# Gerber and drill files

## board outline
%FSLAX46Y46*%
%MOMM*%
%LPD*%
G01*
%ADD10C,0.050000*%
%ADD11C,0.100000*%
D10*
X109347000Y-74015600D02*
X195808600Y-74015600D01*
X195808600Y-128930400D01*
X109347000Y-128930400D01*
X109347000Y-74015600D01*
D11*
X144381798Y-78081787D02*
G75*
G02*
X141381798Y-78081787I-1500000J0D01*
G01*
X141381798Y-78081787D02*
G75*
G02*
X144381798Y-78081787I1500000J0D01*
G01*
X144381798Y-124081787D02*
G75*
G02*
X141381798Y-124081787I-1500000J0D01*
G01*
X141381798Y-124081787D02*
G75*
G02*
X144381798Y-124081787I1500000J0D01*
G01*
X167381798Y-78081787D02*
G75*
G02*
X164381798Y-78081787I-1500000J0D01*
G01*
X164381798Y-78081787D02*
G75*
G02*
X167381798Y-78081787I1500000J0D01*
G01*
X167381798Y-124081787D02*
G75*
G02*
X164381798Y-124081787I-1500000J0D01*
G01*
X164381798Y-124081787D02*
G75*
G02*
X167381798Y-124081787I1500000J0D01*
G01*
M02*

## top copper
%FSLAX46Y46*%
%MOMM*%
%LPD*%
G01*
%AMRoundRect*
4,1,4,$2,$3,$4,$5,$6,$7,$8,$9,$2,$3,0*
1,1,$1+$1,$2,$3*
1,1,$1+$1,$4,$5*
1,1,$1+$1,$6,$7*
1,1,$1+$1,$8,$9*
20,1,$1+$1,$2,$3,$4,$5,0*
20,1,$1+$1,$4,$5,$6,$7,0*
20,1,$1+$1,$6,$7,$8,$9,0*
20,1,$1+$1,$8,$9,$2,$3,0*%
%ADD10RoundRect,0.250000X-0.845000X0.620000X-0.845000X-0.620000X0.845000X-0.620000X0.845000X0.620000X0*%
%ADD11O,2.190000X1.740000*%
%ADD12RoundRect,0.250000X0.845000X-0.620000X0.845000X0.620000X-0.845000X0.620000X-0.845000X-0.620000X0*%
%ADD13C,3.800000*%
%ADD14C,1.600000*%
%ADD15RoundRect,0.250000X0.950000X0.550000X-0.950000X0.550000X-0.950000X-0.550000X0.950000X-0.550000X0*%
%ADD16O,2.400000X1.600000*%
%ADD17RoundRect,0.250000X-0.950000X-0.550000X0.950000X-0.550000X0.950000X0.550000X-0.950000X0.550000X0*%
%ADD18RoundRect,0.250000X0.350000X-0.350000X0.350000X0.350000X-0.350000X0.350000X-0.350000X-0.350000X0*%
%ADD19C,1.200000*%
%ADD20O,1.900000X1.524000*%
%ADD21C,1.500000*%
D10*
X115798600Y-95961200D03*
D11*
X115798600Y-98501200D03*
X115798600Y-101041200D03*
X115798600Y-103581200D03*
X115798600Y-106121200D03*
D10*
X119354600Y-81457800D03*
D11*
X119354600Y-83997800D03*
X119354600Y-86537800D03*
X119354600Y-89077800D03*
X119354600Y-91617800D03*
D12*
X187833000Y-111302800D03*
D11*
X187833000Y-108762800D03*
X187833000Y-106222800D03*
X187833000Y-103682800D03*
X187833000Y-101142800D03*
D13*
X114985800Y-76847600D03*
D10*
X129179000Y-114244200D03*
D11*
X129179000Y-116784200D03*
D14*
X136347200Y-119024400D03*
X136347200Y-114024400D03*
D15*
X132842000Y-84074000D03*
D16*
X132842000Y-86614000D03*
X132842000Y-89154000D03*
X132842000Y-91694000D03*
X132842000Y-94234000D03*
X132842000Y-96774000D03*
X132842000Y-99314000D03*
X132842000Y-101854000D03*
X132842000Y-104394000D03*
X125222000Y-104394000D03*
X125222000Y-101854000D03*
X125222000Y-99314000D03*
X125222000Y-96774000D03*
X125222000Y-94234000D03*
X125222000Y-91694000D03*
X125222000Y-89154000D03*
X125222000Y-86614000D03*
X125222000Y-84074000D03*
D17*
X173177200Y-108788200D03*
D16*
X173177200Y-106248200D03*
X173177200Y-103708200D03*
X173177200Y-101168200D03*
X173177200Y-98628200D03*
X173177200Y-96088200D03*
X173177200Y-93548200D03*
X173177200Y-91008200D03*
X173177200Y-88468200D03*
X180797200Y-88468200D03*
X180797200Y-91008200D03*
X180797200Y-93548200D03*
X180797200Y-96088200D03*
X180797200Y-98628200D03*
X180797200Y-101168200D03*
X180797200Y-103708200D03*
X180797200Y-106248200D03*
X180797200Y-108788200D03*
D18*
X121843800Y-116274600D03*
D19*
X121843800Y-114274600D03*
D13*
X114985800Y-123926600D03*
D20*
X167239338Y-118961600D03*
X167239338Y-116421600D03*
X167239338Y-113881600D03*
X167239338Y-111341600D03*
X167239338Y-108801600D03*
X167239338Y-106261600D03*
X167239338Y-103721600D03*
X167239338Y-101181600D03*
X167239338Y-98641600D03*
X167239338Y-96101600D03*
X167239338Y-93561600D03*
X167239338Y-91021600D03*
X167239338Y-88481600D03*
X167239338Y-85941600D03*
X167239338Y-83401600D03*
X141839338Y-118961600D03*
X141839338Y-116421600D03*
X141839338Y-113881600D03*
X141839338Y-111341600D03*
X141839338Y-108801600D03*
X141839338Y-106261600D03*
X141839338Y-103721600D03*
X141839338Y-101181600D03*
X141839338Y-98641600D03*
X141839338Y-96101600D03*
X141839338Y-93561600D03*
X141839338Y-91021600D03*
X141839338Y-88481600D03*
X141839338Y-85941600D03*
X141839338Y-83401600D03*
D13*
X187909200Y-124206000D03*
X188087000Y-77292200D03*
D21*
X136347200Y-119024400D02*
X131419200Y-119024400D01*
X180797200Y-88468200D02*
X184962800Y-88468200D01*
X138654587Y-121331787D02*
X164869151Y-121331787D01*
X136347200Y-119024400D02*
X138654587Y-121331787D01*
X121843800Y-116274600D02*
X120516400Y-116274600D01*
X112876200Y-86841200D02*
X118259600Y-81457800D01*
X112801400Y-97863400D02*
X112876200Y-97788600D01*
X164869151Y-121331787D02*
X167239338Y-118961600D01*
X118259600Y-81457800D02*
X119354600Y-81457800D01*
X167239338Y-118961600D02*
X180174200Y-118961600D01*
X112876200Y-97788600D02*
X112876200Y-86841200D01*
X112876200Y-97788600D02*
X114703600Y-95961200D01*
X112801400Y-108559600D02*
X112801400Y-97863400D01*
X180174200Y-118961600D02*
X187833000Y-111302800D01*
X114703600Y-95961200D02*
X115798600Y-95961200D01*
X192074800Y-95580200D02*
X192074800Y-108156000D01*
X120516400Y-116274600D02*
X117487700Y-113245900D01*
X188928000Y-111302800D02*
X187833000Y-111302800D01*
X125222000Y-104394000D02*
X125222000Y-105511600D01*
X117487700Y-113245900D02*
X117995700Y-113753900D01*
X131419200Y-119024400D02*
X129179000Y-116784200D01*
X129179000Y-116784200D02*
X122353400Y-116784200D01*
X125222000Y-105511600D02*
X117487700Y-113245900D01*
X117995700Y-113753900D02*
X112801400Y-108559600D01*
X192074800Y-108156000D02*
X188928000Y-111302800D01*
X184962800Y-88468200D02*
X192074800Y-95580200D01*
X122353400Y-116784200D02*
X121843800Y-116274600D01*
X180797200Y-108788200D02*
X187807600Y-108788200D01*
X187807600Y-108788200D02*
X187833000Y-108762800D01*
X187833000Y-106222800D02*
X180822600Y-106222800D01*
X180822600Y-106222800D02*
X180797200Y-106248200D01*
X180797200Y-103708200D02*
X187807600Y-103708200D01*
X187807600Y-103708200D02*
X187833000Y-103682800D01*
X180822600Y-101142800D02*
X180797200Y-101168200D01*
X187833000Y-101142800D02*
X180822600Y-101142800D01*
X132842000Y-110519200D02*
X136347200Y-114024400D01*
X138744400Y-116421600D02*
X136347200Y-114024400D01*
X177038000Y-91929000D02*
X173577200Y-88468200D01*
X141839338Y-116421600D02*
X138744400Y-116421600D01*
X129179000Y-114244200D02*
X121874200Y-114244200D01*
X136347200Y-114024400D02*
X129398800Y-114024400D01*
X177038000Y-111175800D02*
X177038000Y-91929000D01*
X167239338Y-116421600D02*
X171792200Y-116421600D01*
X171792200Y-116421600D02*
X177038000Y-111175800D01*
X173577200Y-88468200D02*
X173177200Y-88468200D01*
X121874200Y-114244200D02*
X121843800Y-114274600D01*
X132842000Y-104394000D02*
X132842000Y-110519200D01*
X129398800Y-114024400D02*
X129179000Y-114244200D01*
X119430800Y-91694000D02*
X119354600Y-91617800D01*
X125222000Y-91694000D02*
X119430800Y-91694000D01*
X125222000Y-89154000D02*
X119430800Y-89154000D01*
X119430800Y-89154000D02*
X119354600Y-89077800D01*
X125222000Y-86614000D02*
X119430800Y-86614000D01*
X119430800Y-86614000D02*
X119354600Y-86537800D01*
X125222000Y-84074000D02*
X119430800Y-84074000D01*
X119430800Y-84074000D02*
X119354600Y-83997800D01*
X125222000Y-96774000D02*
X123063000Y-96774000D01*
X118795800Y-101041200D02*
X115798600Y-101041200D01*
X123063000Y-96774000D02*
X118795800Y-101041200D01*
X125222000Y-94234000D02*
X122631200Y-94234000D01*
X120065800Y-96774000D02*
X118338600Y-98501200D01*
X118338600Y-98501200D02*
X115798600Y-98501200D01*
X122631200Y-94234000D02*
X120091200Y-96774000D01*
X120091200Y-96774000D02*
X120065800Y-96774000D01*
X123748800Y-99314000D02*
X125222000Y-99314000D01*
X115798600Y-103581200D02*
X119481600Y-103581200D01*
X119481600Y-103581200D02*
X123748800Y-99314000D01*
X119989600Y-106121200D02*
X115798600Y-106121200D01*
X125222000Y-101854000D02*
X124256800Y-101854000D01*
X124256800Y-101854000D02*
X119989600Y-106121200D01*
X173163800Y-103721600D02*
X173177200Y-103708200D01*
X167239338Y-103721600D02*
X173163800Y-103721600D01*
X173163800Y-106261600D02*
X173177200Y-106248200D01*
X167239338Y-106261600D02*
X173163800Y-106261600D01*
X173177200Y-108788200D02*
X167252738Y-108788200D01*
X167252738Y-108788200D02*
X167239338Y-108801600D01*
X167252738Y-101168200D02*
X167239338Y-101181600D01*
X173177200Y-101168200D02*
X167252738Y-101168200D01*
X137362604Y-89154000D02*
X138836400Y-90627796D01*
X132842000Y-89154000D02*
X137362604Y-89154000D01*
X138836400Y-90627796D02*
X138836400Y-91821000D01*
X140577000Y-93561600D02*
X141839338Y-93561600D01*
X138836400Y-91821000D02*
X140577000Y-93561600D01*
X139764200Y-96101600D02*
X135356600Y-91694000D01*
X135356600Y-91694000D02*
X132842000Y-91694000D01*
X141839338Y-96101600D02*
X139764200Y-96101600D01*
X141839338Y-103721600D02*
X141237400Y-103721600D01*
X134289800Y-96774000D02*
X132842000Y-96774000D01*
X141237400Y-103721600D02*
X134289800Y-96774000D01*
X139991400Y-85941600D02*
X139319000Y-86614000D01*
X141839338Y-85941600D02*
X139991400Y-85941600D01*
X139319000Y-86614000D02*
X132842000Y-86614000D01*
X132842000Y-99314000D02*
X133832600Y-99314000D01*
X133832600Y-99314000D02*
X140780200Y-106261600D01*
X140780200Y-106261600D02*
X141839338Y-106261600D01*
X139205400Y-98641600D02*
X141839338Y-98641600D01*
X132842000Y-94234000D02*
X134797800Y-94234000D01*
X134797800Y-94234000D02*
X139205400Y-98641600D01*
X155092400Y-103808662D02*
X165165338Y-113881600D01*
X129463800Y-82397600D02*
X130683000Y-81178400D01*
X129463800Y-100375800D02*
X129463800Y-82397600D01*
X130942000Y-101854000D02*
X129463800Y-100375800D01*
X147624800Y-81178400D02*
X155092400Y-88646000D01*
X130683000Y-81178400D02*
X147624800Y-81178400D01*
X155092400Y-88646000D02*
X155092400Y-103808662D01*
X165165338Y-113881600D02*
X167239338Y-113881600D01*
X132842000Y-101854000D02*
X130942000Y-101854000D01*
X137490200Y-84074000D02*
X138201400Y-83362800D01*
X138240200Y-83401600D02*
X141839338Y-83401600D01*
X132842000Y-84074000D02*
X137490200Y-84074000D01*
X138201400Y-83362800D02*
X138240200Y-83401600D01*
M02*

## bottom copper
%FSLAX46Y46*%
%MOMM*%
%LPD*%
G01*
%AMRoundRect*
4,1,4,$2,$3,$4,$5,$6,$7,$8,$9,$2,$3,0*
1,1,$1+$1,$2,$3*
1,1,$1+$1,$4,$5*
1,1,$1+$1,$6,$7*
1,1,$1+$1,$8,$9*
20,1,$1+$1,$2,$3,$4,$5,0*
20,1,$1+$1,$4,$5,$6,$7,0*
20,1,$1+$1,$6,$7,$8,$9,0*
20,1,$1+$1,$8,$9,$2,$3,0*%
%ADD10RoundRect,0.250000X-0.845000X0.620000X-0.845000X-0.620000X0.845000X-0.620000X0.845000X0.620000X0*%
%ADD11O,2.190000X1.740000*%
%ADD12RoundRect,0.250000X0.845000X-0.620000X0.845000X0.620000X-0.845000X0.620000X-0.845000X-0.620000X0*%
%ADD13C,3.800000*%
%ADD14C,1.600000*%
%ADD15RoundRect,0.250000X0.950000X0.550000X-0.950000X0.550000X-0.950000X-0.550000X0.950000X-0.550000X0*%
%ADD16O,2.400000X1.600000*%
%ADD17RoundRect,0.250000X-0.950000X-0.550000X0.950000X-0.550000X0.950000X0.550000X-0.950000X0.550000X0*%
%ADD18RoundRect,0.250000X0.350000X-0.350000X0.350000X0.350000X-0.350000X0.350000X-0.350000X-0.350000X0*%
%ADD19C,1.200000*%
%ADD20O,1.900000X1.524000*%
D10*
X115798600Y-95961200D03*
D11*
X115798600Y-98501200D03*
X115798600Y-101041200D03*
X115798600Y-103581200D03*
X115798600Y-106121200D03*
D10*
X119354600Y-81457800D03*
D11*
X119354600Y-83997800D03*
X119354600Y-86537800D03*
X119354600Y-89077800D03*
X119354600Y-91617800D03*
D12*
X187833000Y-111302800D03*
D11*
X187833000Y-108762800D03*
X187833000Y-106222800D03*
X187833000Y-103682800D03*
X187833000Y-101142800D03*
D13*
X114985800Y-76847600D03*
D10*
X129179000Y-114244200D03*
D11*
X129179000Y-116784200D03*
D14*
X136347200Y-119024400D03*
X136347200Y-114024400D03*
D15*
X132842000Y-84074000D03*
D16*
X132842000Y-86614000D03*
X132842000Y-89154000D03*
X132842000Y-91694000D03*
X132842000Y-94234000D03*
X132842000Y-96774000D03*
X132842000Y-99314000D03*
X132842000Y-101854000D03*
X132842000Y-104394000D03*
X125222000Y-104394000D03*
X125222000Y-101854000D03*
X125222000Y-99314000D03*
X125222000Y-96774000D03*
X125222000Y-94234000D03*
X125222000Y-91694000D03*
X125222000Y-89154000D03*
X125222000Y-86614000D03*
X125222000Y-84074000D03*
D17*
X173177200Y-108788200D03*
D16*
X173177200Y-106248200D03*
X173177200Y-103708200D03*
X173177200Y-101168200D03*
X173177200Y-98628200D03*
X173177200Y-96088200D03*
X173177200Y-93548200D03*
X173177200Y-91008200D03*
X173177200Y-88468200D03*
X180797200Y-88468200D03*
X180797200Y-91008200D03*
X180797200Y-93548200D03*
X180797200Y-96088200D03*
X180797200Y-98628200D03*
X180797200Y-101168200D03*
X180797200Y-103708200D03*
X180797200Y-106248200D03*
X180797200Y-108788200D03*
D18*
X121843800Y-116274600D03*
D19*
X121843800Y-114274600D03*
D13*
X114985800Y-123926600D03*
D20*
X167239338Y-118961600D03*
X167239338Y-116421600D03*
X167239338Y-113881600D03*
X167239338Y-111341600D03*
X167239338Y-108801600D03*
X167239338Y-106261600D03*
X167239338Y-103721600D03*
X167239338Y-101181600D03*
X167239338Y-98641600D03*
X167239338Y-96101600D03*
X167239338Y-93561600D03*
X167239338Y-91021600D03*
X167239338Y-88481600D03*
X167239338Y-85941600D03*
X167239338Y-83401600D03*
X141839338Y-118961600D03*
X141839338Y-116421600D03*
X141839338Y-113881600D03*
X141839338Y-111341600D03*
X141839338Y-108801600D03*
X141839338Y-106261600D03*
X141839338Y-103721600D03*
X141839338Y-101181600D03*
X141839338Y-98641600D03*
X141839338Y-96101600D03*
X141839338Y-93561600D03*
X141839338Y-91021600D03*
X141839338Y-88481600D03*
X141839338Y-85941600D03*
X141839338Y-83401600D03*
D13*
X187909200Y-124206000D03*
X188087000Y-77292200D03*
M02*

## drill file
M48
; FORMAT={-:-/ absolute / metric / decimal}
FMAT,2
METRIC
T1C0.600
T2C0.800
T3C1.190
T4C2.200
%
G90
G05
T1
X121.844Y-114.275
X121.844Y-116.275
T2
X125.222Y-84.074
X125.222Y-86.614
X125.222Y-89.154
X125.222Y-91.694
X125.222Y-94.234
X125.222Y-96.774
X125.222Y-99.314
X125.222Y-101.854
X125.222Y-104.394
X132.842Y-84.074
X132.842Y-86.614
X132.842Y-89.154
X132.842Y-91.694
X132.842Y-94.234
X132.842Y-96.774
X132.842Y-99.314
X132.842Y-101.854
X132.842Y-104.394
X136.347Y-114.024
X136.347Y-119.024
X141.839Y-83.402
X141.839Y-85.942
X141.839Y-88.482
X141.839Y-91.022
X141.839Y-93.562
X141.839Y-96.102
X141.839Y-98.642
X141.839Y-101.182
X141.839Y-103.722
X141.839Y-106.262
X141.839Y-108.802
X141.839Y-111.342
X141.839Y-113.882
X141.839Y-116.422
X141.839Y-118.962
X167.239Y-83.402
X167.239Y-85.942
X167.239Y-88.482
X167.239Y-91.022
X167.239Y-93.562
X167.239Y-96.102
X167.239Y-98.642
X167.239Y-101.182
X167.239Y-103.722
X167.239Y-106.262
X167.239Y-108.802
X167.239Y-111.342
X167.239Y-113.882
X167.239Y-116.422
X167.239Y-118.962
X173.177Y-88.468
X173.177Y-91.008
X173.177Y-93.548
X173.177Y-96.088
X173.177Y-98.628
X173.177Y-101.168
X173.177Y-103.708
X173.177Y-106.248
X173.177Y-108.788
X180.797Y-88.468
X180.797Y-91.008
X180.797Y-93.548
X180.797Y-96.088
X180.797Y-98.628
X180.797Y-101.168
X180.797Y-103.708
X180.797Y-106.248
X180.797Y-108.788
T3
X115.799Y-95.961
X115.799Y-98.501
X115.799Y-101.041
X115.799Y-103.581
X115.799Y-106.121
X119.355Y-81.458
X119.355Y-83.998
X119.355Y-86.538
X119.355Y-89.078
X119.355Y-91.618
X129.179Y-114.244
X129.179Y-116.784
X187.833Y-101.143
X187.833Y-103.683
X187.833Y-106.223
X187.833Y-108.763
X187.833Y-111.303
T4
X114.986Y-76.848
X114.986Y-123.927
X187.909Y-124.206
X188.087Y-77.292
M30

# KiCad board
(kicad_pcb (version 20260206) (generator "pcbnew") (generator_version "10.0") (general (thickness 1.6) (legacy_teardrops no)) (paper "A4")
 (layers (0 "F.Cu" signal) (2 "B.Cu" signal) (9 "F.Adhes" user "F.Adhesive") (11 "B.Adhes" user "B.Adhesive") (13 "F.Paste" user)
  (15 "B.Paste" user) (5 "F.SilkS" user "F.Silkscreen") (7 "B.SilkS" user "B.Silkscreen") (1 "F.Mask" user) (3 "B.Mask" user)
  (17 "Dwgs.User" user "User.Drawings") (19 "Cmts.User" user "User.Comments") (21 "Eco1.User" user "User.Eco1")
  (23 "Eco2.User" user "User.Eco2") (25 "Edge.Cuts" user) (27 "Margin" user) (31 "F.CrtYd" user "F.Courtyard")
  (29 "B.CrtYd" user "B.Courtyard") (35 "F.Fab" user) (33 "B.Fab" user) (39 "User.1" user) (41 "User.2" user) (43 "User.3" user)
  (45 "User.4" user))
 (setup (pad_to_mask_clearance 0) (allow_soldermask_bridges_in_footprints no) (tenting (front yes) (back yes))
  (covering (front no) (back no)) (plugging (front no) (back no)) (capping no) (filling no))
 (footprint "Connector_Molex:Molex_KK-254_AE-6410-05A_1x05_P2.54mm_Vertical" (layer "F.Cu") (at 115.7986 95.9612 -90)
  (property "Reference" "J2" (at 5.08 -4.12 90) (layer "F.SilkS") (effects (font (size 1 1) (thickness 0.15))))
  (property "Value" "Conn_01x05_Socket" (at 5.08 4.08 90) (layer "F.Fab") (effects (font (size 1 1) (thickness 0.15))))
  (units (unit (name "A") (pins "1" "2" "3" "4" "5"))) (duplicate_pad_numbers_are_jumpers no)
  (pad "1" thru_hole roundrect (at 0 0 270) (size 1.74 2.19) (drill 1.19) (layers "*.Cu" "*.Mask") (remove_unused_layers no)
   (roundrect_rratio 0.143678) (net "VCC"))
  (pad "2" thru_hole oval (at 2.54 0 270) (size 1.74 2.19) (drill 1.19) (layers "*.Cu" "*.Mask") (remove_unused_layers no)
   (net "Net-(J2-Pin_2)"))
  (pad "3" thru_hole oval (at 5.08 0 270) (size 1.74 2.19) (drill 1.19) (layers "*.Cu" "*.Mask") (remove_unused_layers no)
   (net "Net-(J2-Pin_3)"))
  (pad "4" thru_hole oval (at 7.62 0 270) (size 1.74 2.19) (drill 1.19) (layers "*.Cu" "*.Mask") (remove_unused_layers no)
   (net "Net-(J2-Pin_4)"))
  (pad "5" thru_hole oval (at 10.16 0 270) (size 1.74 2.19) (drill 1.19) (layers "*.Cu" "*.Mask") (remove_unused_layers no)
   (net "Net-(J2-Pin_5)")))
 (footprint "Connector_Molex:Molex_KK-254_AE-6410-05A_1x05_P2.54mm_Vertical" (layer "F.Cu") (at 119.3546 81.4578 -90)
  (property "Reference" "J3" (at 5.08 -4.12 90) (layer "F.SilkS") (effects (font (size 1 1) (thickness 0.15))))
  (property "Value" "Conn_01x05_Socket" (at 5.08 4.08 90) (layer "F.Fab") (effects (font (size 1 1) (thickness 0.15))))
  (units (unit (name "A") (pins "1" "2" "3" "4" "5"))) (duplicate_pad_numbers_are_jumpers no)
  (pad "1" thru_hole roundrect (at 0 0 270) (size 1.74 2.19) (drill 1.19) (layers "*.Cu" "*.Mask") (remove_unused_layers no)
   (roundrect_rratio 0.143678) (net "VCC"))
  (pad "2" thru_hole oval (at 2.54 0 270) (size 1.74 2.19) (drill 1.19) (layers "*.Cu" "*.Mask") (remove_unused_layers no) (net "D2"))
  (pad "3" thru_hole oval (at 5.08 0 270) (size 1.74 2.19) (drill 1.19) (layers "*.Cu" "*.Mask") (remove_unused_layers no) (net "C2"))
  (pad "4" thru_hole oval (at 7.62 0 270) (size 1.74 2.19) (drill 1.19) (layers "*.Cu" "*.Mask") (remove_unused_layers no) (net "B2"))
  (pad "5" thru_hole oval (at 10.16 0 270) (size 1.74 2.19) (drill 1.19) (layers "*.Cu" "*.Mask") (remove_unused_layers no) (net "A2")))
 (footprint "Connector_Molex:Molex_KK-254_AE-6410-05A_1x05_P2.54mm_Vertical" (layer "B.Cu") (at 187.833 111.3028 90)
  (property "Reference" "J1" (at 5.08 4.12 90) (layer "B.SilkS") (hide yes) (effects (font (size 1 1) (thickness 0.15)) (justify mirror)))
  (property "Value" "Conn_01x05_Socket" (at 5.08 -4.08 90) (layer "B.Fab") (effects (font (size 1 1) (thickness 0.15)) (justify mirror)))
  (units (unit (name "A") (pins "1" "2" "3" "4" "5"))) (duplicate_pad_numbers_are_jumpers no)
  (pad "1" thru_hole roundrect (at 0 0 90) (size 1.74 2.19) (drill 1.19) (layers "*.Cu" "*.Mask") (remove_unused_layers no)
   (roundrect_rratio 0.143678) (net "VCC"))
  (pad "2" thru_hole oval (at 2.54 0 90) (size 1.74 2.19) (drill 1.19) (layers "*.Cu" "*.Mask") (remove_unused_layers no) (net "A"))
  (pad "3" thru_hole oval (at 5.08 0 90) (size 1.74 2.19) (drill 1.19) (layers "*.Cu" "*.Mask") (remove_unused_layers no) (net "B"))
  (pad "4" thru_hole oval (at 7.62 0 90) (size 1.74 2.19) (drill 1.19) (layers "*.Cu" "*.Mask") (remove_unused_layers no) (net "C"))
  (pad "5" thru_hole oval (at 10.16 0 90) (size 1.74 2.19) (drill 1.19) (layers "*.Cu" "*.Mask") (remove_unused_layers no) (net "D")))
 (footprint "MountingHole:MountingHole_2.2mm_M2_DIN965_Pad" (layer "B.Cu") (at 114.9858 76.8476 90)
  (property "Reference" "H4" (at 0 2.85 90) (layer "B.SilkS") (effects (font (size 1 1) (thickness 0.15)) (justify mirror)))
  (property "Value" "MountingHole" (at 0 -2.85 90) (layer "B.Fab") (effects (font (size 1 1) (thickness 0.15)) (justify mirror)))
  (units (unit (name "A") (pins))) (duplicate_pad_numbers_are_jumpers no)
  (pad "1" thru_hole circle (at 0 0 90) (size 3.8 3.8) (drill 2.2) (layers "*.Cu" "*.Mask") (remove_unused_layers no) (zone_connect 2)))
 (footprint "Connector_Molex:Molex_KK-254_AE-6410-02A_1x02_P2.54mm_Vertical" (layer "B.Cu") (at 129.179 114.2442 -90)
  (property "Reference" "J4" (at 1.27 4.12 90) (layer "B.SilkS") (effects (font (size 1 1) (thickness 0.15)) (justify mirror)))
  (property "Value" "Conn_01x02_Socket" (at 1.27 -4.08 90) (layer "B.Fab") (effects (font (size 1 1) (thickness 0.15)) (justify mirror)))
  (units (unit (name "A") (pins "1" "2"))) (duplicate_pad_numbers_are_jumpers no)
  (pad "1" thru_hole roundrect (at 0 0 270) (size 1.74 2.19) (drill 1.19) (layers "*.Cu" "*.Mask") (remove_unused_layers no)
   (roundrect_rratio 0.143678) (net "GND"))
  (pad "2" thru_hole oval (at 2.54 0 270) (size 1.74 2.19) (drill 1.19) (layers "*.Cu" "*.Mask") (remove_unused_layers no) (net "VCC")))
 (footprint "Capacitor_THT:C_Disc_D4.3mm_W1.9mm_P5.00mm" (layer "B.Cu") (at 136.3472 119.0244 90)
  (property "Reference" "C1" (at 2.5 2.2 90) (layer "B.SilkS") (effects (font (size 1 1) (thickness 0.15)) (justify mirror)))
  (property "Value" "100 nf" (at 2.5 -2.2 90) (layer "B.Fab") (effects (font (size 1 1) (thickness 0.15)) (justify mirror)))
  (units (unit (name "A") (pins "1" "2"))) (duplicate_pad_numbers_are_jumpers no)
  (pad "1" thru_hole circle (at 0 0 90) (size 1.6 1.6) (drill 0.8) (layers "*.Cu" "*.Mask") (remove_unused_layers no) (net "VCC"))
  (pad "2" thru_hole circle (at 5 0 90) (size 1.6 1.6) (drill 0.8) (layers "*.Cu" "*.Mask") (remove_unused_layers no) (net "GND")))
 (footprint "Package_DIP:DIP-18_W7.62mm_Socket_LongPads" (layer "B.Cu") (at 132.842 84.074 180)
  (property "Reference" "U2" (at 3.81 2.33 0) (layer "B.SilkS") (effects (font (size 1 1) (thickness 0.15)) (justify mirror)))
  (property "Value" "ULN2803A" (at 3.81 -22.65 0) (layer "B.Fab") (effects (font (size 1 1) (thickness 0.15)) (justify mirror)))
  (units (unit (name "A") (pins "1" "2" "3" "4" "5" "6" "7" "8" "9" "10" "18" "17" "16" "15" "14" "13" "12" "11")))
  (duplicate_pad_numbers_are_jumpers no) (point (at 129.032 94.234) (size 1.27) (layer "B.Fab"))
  (pad "1" thru_hole roundrect (at 0 0 180) (size 2.4 1.6) (drill 0.8) (layers "*.Cu" "*.Mask") (remove_unused_layers no)
   (roundrect_rratio 0.15625) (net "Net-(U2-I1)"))
  (pad "2" thru_hole oval (at 0 -2.54 180) (size 2.4 1.6) (drill 0.8) (layers "*.Cu" "*.Mask") (remove_unused_layers no) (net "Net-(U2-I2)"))
  (pad "3" thru_hole oval (at 0 -5.08 180) (size 2.4 1.6) (drill 0.8) (layers "*.Cu" "*.Mask") (remove_unused_layers no) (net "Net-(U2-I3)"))
  (pad "4" thru_hole oval (at 0 -7.62 180) (size 2.4 1.6) (drill 0.8) (layers "*.Cu" "*.Mask") (remove_unused_layers no) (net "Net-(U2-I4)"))
  (pad "5" thru_hole oval (at 0 -10.16 180) (size 2.4 1.6) (drill 0.8) (layers "*.Cu" "*.Mask") (remove_unused_layers no)
   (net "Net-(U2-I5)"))
  (pad "6" thru_hole oval (at 0 -12.7 180) (size 2.4 1.6) (drill 0.8) (layers "*.Cu" "*.Mask") (remove_unused_layers no) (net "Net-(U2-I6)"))
  (pad "7" thru_hole oval (at 0 -15.24 180) (size 2.4 1.6) (drill 0.8) (layers "*.Cu" "*.Mask") (remove_unused_layers no)
   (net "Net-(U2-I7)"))
  (pad "8" thru_hole oval (at 0 -17.78 180) (size 2.4 1.6) (drill 0.8) (layers "*.Cu" "*.Mask") (remove_unused_layers no)
   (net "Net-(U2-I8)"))
  (pad "9" thru_hole oval (at 0 -20.32 180) (size 2.4 1.6) (drill 0.8) (layers "*.Cu" "*.Mask") (remove_unused_layers no) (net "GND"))
  (pad "10" thru_hole oval (at 7.62 -20.32 180) (size 2.4 1.6) (drill 0.8) (layers "*.Cu" "*.Mask") (remove_unused_layers no) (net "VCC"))
  (pad "11" thru_hole oval (at 7.62 -17.78 180) (size 2.4 1.6) (drill 0.8) (layers "*.Cu" "*.Mask") (remove_unused_layers no)
   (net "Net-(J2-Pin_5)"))
  (pad "12" thru_hole oval (at 7.62 -15.24 180) (size 2.4 1.6) (drill 0.8) (layers "*.Cu" "*.Mask") (remove_unused_layers no)
   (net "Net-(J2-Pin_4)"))
  (pad "13" thru_hole oval (at 7.62 -12.7 180) (size 2.4 1.6) (drill 0.8) (layers "*.Cu" "*.Mask") (remove_unused_layers no)
   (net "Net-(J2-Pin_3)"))
  (pad "14" thru_hole oval (at 7.62 -10.16 180) (size 2.4 1.6) (drill 0.8) (layers "*.Cu" "*.Mask") (remove_unused_layers no)
   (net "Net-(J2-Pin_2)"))
  (pad "15" thru_hole oval (at 7.62 -7.62 180) (size 2.4 1.6) (drill 0.8) (layers "*.Cu" "*.Mask") (remove_unused_layers no) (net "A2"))
  (pad "16" thru_hole oval (at 7.62 -5.08 180) (size 2.4 1.6) (drill 0.8) (layers "*.Cu" "*.Mask") (remove_unused_layers no) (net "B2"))
  (pad "17" thru_hole oval (at 7.62 -2.54 180) (size 2.4 1.6) (drill 0.8) (layers "*.Cu" "*.Mask") (remove_unused_layers no) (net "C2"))
  (pad "18" thru_hole oval (at 7.62 0 180) (size 2.4 1.6) (drill 0.8) (layers "*.Cu" "*.Mask") (remove_unused_layers no) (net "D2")))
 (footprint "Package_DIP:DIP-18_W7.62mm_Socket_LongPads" (layer "B.Cu") (at 173.1772 108.7882)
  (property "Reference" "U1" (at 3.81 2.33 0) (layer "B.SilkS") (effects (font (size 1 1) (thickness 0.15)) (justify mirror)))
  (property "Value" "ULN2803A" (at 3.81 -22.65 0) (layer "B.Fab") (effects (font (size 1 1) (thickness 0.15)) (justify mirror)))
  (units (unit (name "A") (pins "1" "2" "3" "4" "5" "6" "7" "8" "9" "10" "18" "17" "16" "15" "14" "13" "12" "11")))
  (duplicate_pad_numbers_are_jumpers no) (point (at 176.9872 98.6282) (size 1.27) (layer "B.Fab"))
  (pad "1" thru_hole roundrect (at 0 0) (size 2.4 1.6) (drill 0.8) (layers "*.Cu" "*.Mask") (remove_unused_layers no)
   (roundrect_rratio 0.15625) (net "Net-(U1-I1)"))
  (pad "2" thru_hole oval (at 0 -2.54) (size 2.4 1.6) (drill 0.8) (layers "*.Cu" "*.Mask") (remove_unused_layers no) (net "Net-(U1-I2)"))
  (pad "3" thru_hole oval (at 0 -5.08) (size 2.4 1.6) (drill 0.8) (layers "*.Cu" "*.Mask") (remove_unused_layers no) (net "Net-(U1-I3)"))
  (pad "4" thru_hole oval (at 0 -7.62) (size 2.4 1.6) (drill 0.8) (layers "*.Cu" "*.Mask") (remove_unused_layers no) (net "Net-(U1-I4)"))
  (pad "5" thru_hole oval (at 0 -10.16) (size 2.4 1.6) (drill 0.8) (layers "*.Cu" "*.Mask") (remove_unused_layers no)
   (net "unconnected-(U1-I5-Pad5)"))
  (pad "6" thru_hole oval (at 0 -12.7) (size 2.4 1.6) (drill 0.8) (layers "*.Cu" "*.Mask") (remove_unused_layers no)
   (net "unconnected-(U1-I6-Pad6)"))
  (pad "7" thru_hole oval (at 0 -15.24) (size 2.4 1.6) (drill 0.8) (layers "*.Cu" "*.Mask") (remove_unused_layers no)
   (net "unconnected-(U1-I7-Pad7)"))
  (pad "8" thru_hole oval (at 0 -17.78) (size 2.4 1.6) (drill 0.8) (layers "*.Cu" "*.Mask") (remove_unused_layers no)
   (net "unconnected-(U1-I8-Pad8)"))
  (pad "9" thru_hole oval (at 0 -20.32) (size 2.4 1.6) (drill 0.8) (layers "*.Cu" "*.Mask") (remove_unused_layers no) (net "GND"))
  (pad "10" thru_hole oval (at 7.62 -20.32) (size 2.4 1.6) (drill 0.8) (layers "*.Cu" "*.Mask") (remove_unused_layers no) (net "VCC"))
  (pad "11" thru_hole oval (at 7.62 -17.78) (size 2.4 1.6) (drill 0.8) (layers "*.Cu" "*.Mask") (remove_unused_layers no)
   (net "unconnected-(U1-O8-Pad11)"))
  (pad "12" thru_hole oval (at 7.62 -15.24) (size 2.4 1.6) (drill 0.8) (layers "*.Cu" "*.Mask") (remove_unused_layers no)
   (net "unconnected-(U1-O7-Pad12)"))
  (pad "13" thru_hole oval (at 7.62 -12.7) (size 2.4 1.6) (drill 0.8) (layers "*.Cu" "*.Mask") (remove_unused_layers no)
   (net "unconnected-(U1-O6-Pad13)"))
  (pad "14" thru_hole oval (at 7.62 -10.16) (size 2.4 1.6) (drill 0.8) (layers "*.Cu" "*.Mask") (remove_unused_layers no)
   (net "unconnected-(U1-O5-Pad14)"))
  (pad "15" thru_hole oval (at 7.62 -7.62) (size 2.4 1.6) (drill 0.8) (layers "*.Cu" "*.Mask") (remove_unused_layers no) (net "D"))
  (pad "16" thru_hole oval (at 7.62 -5.08) (size 2.4 1.6) (drill 0.8) (layers "*.Cu" "*.Mask") (remove_unused_layers no) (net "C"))
  (pad "17" thru_hole oval (at 7.62 -2.54) (size 2.4 1.6) (drill 0.8) (layers "*.Cu" "*.Mask") (remove_unused_layers no) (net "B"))
  (pad "18" thru_hole oval (at 7.62 0) (size 2.4 1.6) (drill 0.8) (layers "*.Cu" "*.Mask") (remove_unused_layers no) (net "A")))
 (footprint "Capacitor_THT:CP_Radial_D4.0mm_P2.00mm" (layer "B.Cu") (at 121.8438 116.2746 90)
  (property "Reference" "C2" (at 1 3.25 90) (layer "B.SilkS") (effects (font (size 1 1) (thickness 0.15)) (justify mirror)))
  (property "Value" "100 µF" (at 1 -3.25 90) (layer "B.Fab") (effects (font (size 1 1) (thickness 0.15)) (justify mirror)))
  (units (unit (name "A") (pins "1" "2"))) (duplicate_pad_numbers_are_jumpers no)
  (pad "1" thru_hole roundrect (at 0 0 90) (size 1.2 1.2) (drill 0.6) (layers "*.Cu" "*.Mask") (remove_unused_layers no)
   (roundrect_rratio 0.208333) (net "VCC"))
  (pad "2" thru_hole circle (at 2 0 90) (size 1.2 1.2) (drill 0.6) (layers "*.Cu" "*.Mask") (remove_unused_layers no) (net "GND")))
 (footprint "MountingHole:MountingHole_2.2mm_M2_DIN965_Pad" (layer "B.Cu") (at 114.9858 123.9266 90)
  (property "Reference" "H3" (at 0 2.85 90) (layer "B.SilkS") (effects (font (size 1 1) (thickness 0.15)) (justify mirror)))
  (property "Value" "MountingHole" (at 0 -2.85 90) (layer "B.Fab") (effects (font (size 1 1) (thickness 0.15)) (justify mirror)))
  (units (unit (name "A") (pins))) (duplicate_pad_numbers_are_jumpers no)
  (pad "1" thru_hole circle (at 0 0 90) (size 3.8 3.8) (drill 2.2) (layers "*.Cu" "*.Mask") (remove_unused_layers no) (zone_connect 2)))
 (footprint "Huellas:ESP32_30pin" (layer "B.Cu") (at 155.311798 101.941787 180)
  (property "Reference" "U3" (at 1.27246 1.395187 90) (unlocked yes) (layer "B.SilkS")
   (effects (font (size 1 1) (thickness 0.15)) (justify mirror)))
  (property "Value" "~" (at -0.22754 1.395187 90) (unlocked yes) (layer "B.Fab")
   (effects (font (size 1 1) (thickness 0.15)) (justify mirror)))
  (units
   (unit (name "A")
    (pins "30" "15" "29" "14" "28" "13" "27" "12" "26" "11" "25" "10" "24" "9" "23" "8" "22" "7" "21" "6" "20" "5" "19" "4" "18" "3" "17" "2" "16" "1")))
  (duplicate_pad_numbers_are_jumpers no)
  (fp_circle (center 12.43 23.86) (end 12.43 22.36) (stroke (width 0.1) (type default)) (fill no) (layer "Edge.Cuts"))
  (fp_circle (center 12.43 -22.14) (end 12.43 -23.64) (stroke (width 0.1) (type default)) (fill no) (layer "Edge.Cuts"))
  (fp_circle (center -10.57 23.86) (end -10.57 22.36) (stroke (width 0.1) (type default)) (fill no) (layer "Edge.Cuts"))
  (fp_circle (center -10.57 -22.14) (end -10.57 -23.64) (stroke (width 0.1) (type default)) (fill no) (layer "Edge.Cuts"))
  (pad "1" thru_hole oval (at -11.92754 -17.019813 270) (size 1.524 1.9) (drill 0.8) (layers "*.Cu" "*.Mask") (remove_unused_layers no)
   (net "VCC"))
  (pad "2" thru_hole oval (at -11.92754 -14.479813 270) (size 1.524 1.9) (drill 0.8) (layers "*.Cu" "*.Mask") (remove_unused_layers no)
   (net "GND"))
  (pad "3" thru_hole oval (at -11.92754 -11.939813 270) (size 1.524 1.9) (drill 0.8) (layers "*.Cu" "*.Mask") (remove_unused_layers no)
   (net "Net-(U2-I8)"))
  (pad "4" thru_hole oval (at -11.92754 -9.399813 270) (size 1.524 1.9) (drill 0.8) (layers "*.Cu" "*.Mask") (remove_unused_layers no)
   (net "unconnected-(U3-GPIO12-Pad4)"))
  (pad "5" thru_hole oval (at -11.92754 -6.859813 270) (size 1.524 1.9) (drill 0.8) (layers "*.Cu" "*.Mask") (remove_unused_layers no)
   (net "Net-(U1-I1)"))
  (pad "6" thru_hole oval (at -11.92754 -4.319813 270) (size 1.524 1.9) (drill 0.8) (layers "*.Cu" "*.Mask") (remove_unused_layers no)
   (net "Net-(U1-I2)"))
  (pad "7" thru_hole oval (at -11.92754 -1.779813 270) (size 1.524 1.9) (drill 0.8) (layers "*.Cu" "*.Mask") (remove_unused_layers no)
   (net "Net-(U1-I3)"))
  (pad "8" thru_hole oval (at -11.92754 0.760187 270) (size 1.524 1.9) (drill 0.8) (layers "*.Cu" "*.Mask") (remove_unused_layers no)
   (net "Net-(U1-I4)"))
  (pad "9" thru_hole oval (at -11.92754 3.300187 270) (size 1.524 1.9) (drill 0.8) (layers "*.Cu" "*.Mask") (remove_unused_layers no)
   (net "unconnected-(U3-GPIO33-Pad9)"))
  (pad "10" thru_hole oval (at -11.92754 5.840187 270) (size 1.524 1.9) (drill 0.8) (layers "*.Cu" "*.Mask") (remove_unused_layers no)
   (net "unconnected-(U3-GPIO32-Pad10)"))
  (pad "11" thru_hole oval (at -11.92754 8.380187 270) (size 1.524 1.9) (drill 0.8) (layers "*.Cu" "*.Mask") (remove_unused_layers no)
   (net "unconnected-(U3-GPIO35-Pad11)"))
  (pad "12" thru_hole oval (at -11.92754 10.920187 270) (size 1.524 1.9) (drill 0.8) (layers "*.Cu" "*.Mask") (remove_unused_layers no)
   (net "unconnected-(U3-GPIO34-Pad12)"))
  (pad "13" thru_hole oval (at -11.92754 13.460187 270) (size 1.524 1.9) (drill 0.8) (layers "*.Cu" "*.Mask") (remove_unused_layers no)
   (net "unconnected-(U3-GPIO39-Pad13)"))
  (pad "14" thru_hole oval (at -11.92754 16.000187 270) (size 1.524 1.9) (drill 0.8) (layers "*.Cu" "*.Mask") (remove_unused_layers no)
   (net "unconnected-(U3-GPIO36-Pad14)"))
  (pad "15" thru_hole oval (at -11.92754 18.540187 270) (size 1.524 1.9) (drill 0.8) (layers "*.Cu" "*.Mask") (remove_unused_layers no)
   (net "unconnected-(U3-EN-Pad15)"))
  (pad "16" thru_hole oval (at 13.47246 -17.019813 270) (size 1.524 1.9) (drill 0.8) (layers "*.Cu" "*.Mask") (remove_unused_layers no)
   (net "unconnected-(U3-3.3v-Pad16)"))
  (pad "17" thru_hole oval (at 13.47246 -14.479813 270) (size 1.524 1.9) (drill 0.8) (layers "*.Cu" "*.Mask") (remove_unused_layers no)
   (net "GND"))
  (pad "18" thru_hole oval (at 13.47246 -11.939813 270) (size 1.524 1.9) (drill 0.8) (layers "*.Cu" "*.Mask") (remove_unused_layers no)
   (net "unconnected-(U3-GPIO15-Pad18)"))
  (pad "19" thru_hole oval (at 13.47246 -9.399813 270) (size 1.524 1.9) (drill 0.8) (layers "*.Cu" "*.Mask") (remove_unused_layers no)
   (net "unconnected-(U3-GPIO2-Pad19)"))
  (pad "20" thru_hole oval (at 13.47246 -6.859813 270) (size 1.524 1.9) (drill 0.8) (layers "*.Cu" "*.Mask" "Dwgs.User")
   (remove_unused_layers no) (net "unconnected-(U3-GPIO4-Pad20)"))
  (pad "21" thru_hole oval (at 13.47246 -4.319813 270) (size 1.524 1.9) (drill 0.8) (layers "*.Cu" "*.Mask") (remove_unused_layers no)
   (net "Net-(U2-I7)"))
  (pad "22" thru_hole oval (at 13.47246 -1.779813 270) (size 1.524 1.9) (drill 0.8) (layers "*.Cu" "*.Mask") (remove_unused_layers no)
   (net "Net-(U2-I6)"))
  (pad "23" thru_hole oval (at 13.47246 0.760187 270) (size 1.524 1.9) (drill 0.8) (layers "*.Cu" "*.Mask") (remove_unused_layers no)
   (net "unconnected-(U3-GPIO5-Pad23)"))
  (pad "24" thru_hole oval (at 13.47246 3.300187 270) (size 1.524 1.9) (drill 0.8) (layers "*.Cu" "*.Mask") (remove_unused_layers no)
   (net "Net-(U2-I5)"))
  (pad "25" thru_hole oval (at 13.47246 5.840187 270) (size 1.524 1.9) (drill 0.8) (layers "*.Cu" "*.Mask") (remove_unused_layers no)
   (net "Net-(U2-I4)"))
  (pad "26" thru_hole oval (at 13.47246 8.380187 270) (size 1.524 1.9) (drill 0.8) (layers "*.Cu" "*.Mask") (remove_unused_layers no)
   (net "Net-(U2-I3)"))
  (pad "27" thru_hole oval (at 13.47246 10.920187 270) (size 1.524 1.9) (drill 0.8) (layers "*.Cu" "*.Mask") (remove_unused_layers no)
   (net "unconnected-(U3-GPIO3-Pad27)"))
  (pad "28" thru_hole oval (at 13.47246 13.460187 270) (size 1.524 1.9) (drill 0.8) (layers "*.Cu" "*.Mask") (remove_unused_layers no)
   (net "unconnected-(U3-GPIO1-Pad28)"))
  (pad "29" thru_hole oval (at 13.47246 16.000187 270) (size 1.524 1.9) (drill 0.8) (layers "*.Cu" "*.Mask") (remove_unused_layers no)
   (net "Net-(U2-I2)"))
  (pad "30" thru_hole oval (at 13.47246 18.540187 270) (size 1.524 1.9) (drill 0.8) (layers "*.Cu" "*.Mask") (remove_unused_layers no)
   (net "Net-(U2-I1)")))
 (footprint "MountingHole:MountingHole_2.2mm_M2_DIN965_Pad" (layer "B.Cu") (at 187.9092 124.206 90)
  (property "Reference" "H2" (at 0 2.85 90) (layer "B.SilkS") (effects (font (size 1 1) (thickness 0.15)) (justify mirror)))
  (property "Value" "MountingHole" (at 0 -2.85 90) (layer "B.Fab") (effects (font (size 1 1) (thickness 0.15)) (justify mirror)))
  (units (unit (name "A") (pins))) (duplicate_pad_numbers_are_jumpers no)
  (pad "1" thru_hole circle (at 0 0 90) (size 3.8 3.8) (drill 2.2) (layers "*.Cu" "*.Mask") (remove_unused_layers no) (zone_connect 2)))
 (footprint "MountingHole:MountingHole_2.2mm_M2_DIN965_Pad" (layer "B.Cu") (at 188.087 77.2922 90)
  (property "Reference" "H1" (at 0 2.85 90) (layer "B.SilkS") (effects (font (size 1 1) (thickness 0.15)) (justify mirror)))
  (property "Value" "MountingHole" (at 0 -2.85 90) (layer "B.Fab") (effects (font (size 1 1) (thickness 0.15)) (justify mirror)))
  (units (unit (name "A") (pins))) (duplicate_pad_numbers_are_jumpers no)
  (pad "1" thru_hole circle (at 0 0 90) (size 3.8 3.8) (drill 2.2) (layers "*.Cu" "*.Mask") (remove_unused_layers no) (zone_connect 2)))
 (gr_rect (start 109.347 74.0156) (end 195.8086 128.9304) (stroke (width 0.05) (type default)) (fill no) (layer "Edge.Cuts"))
 (segment (start 136.3472 119.0244) (end 131.4192 119.0244) (width 1.5) (layer "F.Cu") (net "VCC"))
 (segment (start 180.7972 88.4682) (end 184.9628 88.4682) (width 1.5) (layer "F.Cu") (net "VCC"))
 (segment (start 138.654587 121.331787) (end 164.869151 121.331787) (width 1.5) (layer "F.Cu") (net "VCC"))
 (segment (start 136.3472 119.0244) (end 138.654587 121.331787) (width 1.5) (layer "F.Cu") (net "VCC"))
 (segment (start 121.8438 116.2746) (end 120.5164 116.2746) (width 1.5) (layer "F.Cu") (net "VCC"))
 (segment (start 112.8762 86.8412) (end 118.2596 81.4578) (width 1.5) (layer "F.Cu") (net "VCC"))
 (segment (start 112.8014 97.8634) (end 112.8762 97.7886) (width 1.5) (layer "F.Cu") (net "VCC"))
 (segment (start 164.869151 121.331787) (end 167.239338 118.9616) (width 1.5) (layer "F.Cu") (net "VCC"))
 (segment (start 118.2596 81.4578) (end 119.3546 81.4578) (width 1.5) (layer "F.Cu") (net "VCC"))
 (segment (start 167.239338 118.9616) (end 180.1742 118.9616) (width 1.5) (layer "F.Cu") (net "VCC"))
 (segment (start 112.8762 97.7886) (end 112.8762 86.8412) (width 1.5) (layer "F.Cu") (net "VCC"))
 (segment (start 112.8762 97.7886) (end 114.7036 95.9612) (width 1.5) (layer "F.Cu") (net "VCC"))
 (segment (start 112.8014 108.5596) (end 112.8014 97.8634) (width 1.5) (layer "F.Cu") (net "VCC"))
 (segment (start 180.1742 118.9616) (end 187.833 111.3028) (width 1.5) (layer "F.Cu") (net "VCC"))
 (segment (start 114.7036 95.9612) (end 115.7986 95.9612) (width 1.5) (layer "F.Cu") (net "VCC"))
 (segment (start 192.0748 95.5802) (end 192.0748 108.156) (width 1.5) (layer "F.Cu") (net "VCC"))
 (segment (start 120.5164 116.2746) (end 117.4877 113.2459) (width 1.5) (layer "F.Cu") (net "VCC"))
 (segment (start 188.928 111.3028) (end 187.833 111.3028) (width 1.5) (layer "F.Cu") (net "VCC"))
 (segment (start 125.222 104.394) (end 125.222 105.5116) (width 1.5) (layer "F.Cu") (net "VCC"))
 (segment (start 117.4877 113.2459) (end 117.9957 113.7539) (width 1.5) (layer "F.Cu") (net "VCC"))
 (segment (start 131.4192 119.0244) (end 129.179 116.7842) (width 1.5) (layer "F.Cu") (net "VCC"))
 (segment (start 129.179 116.7842) (end 122.3534 116.7842) (width 1.5) (layer "F.Cu") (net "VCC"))
 (segment (start 125.222 105.5116) (end 117.4877 113.2459) (width 1.5) (layer "F.Cu") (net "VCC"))
 (segment (start 117.9957 113.7539) (end 112.8014 108.5596) (width 1.5) (layer "F.Cu") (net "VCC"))
 (segment (start 192.0748 108.156) (end 188.928 111.3028) (width 1.5) (layer "F.Cu") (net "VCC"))
 (segment (start 184.9628 88.4682) (end 192.0748 95.5802) (width 1.5) (layer "F.Cu") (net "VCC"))
 (segment (start 122.3534 116.7842) (end 121.8438 116.2746) (width 1.5) (layer "F.Cu") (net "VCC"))
 (segment (start 180.7972 108.7882) (end 187.8076 108.7882) (width 1.5) (layer "F.Cu") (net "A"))
 (segment (start 187.8076 108.7882) (end 187.833 108.7628) (width 1.5) (layer "F.Cu") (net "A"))
 (segment (start 187.833 106.2228) (end 180.8226 106.2228) (width 1.5) (layer "F.Cu") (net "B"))
 (segment (start 180.8226 106.2228) (end 180.7972 106.2482) (width 1.5) (layer "F.Cu") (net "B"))
 (segment (start 180.7972 103.7082) (end 187.8076 103.7082) (width 1.5) (layer "F.Cu") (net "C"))
 (segment (start 187.8076 103.7082) (end 187.833 103.6828) (width 1.5) (layer "F.Cu") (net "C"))
 (segment (start 180.8226 101.1428) (end 180.7972 101.1682) (width 1.5) (layer "F.Cu") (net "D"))
 (segment (start 187.833 101.1428) (end 180.8226 101.1428) (width 1.5) (layer "F.Cu") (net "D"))
 (segment (start 132.842 110.5192) (end 136.3472 114.0244) (width 1.5) (layer "F.Cu") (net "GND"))
 (segment (start 138.7444 116.4216) (end 136.3472 114.0244) (width 1.5) (layer "F.Cu") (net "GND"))
 (segment (start 177.038 91.929) (end 173.5772 88.4682) (width 1.5) (layer "F.Cu") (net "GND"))
 (segment (start 141.839338 116.4216) (end 138.7444 116.4216) (width 1.5) (layer "F.Cu") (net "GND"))
 (segment (start 129.179 114.2442) (end 121.8742 114.2442) (width 1.5) (layer "F.Cu") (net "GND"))
 (segment (start 136.3472 114.0244) (end 129.3988 114.0244) (width 1.5) (layer "F.Cu") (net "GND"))
 (segment (start 177.038 111.1758) (end 177.038 91.929) (width 1.5) (layer "F.Cu") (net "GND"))
 (segment (start 167.239338 116.4216) (end 171.7922 116.4216) (width 1.5) (layer "F.Cu") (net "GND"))
 (segment (start 171.7922 116.4216) (end 177.038 111.1758) (width 1.5) (layer "F.Cu") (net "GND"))
 (segment (start 173.5772 88.4682) (end 173.1772 88.4682) (width 1.5) (layer "F.Cu") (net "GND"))
 (segment (start 121.8742 114.2442) (end 121.8438 114.2746) (width 1.5) (layer "F.Cu") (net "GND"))
 (segment (start 132.842 104.394) (end 132.842 110.5192) (width 1.5) (layer "F.Cu") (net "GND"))
 (segment (start 129.3988 114.0244) (end 129.179 114.2442) (width 1.5) (layer "F.Cu") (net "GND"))
 (segment (start 119.4308 91.694) (end 119.3546 91.6178) (width 1.5) (layer "F.Cu") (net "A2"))
 (segment (start 125.222 91.694) (end 119.4308 91.694) (width 1.5) (layer "F.Cu") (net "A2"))
 (segment (start 125.222 89.154) (end 119.4308 89.154) (width 1.5) (layer "F.Cu") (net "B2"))
 (segment (start 119.4308 89.154) (end 119.3546 89.0778) (width 1.5) (layer "F.Cu") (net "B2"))
 (segment (start 125.222 86.614) (end 119.4308 86.614) (width 1.5) (layer "F.Cu") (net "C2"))
 (segment (start 119.4308 86.614) (end 119.3546 86.5378) (width 1.5) (layer "F.Cu") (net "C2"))
 (segment (start 125.222 84.074) (end 119.4308 84.074) (width 1.5) (layer "F.Cu") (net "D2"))
 (segment (start 119.4308 84.074) (end 119.3546 83.9978) (width 1.5) (layer "F.Cu") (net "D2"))
 (segment (start 125.222 96.774) (end 123.063 96.774) (width 1.5) (layer "F.Cu") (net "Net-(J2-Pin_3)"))
 (segment (start 118.7958 101.0412) (end 115.7986 101.0412) (width 1.5) (layer "F.Cu") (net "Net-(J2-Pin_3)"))
 (segment (start 123.063 96.774) (end 118.7958 101.0412) (width 1.5) (layer "F.Cu") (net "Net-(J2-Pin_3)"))
 (segment (start 125.222 94.234) (end 122.6312 94.234) (width 1.5) (layer "F.Cu") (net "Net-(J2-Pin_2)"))
 (segment (start 120.0658 96.774) (end 118.3386 98.5012) (width 1.5) (layer "F.Cu") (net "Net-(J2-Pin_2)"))
 (segment (start 118.3386 98.5012) (end 115.7986 98.5012) (width 1.5) (layer "F.Cu") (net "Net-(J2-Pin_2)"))
 (segment (start 122.6312 94.234) (end 120.0912 96.774) (width 1.5) (layer "F.Cu") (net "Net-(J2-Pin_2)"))
 (segment (start 120.0912 96.774) (end 120.0658 96.774) (width 1.5) (layer "F.Cu") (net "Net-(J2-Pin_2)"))
 (segment (start 123.7488 99.314) (end 125.222 99.314) (width 1.5) (layer "F.Cu") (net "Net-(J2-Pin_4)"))
 (segment (start 115.7986 103.5812) (end 119.4816 103.5812) (width 1.5) (layer "F.Cu") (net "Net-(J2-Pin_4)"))
 (segment (start 119.4816 103.5812) (end 123.7488 99.314) (width 1.5) (layer "F.Cu") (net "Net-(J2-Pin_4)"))
 (segment (start 119.9896 106.1212) (end 115.7986 106.1212) (width 1.5) (layer "F.Cu") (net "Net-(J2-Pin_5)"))
 (segment (start 125.222 101.854) (end 124.2568 101.854) (width 1.5) (layer "F.Cu") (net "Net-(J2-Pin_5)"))
 (segment (start 124.2568 101.854) (end 119.9896 106.1212) (width 1.5) (layer "F.Cu") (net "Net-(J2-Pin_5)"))
 (segment (start 173.1638 103.7216) (end 173.1772 103.7082) (width 1.5) (layer "F.Cu") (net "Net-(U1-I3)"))
 (segment (start 167.239338 103.7216) (end 173.1638 103.7216) (width 1.5) (layer "F.Cu") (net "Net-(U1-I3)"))
 (segment (start 173.1638 106.2616) (end 173.1772 106.2482) (width 1.5) (layer "F.Cu") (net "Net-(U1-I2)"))
 (segment (start 167.239338 106.2616) (end 173.1638 106.2616) (width 1.5) (layer "F.Cu") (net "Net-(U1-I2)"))
 (segment (start 173.1772 108.7882) (end 167.252738 108.7882) (width 1.5) (layer "F.Cu") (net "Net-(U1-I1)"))
 (segment (start 167.252738 108.7882) (end 167.239338 108.8016) (width 1.5) (layer "F.Cu") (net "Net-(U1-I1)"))
 (segment (start 167.252738 101.1682) (end 167.239338 101.1816) (width 1.5) (layer "F.Cu") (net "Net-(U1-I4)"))
 (segment (start 173.1772 101.1682) (end 167.252738 101.1682) (width 1.5) (layer "F.Cu") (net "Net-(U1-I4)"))
 (segment (start 137.362604 89.154) (end 138.8364 90.627796) (width 1.5) (layer "F.Cu") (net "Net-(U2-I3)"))
 (segment (start 132.842 89.154) (end 137.362604 89.154) (width 1.5) (layer "F.Cu") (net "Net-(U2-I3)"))
 (segment (start 138.8364 90.627796) (end 138.8364 91.821) (width 1.5) (layer "F.Cu") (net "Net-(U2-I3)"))
 (segment (start 140.577 93.5616) (end 141.839338 93.5616) (width 1.5) (layer "F.Cu") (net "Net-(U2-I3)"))
 (segment (start 138.8364 91.821) (end 140.577 93.5616) (width 1.5) (layer "F.Cu") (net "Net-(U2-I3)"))
 (segment (start 139.7642 96.1016) (end 135.3566 91.694) (width 1.5) (layer "F.Cu") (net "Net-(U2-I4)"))
 (segment (start 135.3566 91.694) (end 132.842 91.694) (width 1.5) (layer "F.Cu") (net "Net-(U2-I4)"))
 (segment (start 141.839338 96.1016) (end 139.7642 96.1016) (width 1.5) (layer "F.Cu") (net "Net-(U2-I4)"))
 (segment (start 141.839338 103.7216) (end 141.2374 103.7216) (width 1.5) (layer "F.Cu") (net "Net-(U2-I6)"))
 (segment (start 134.2898 96.774) (end 132.842 96.774) (width 1.5) (layer "F.Cu") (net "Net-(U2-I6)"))
 (segment (start 141.2374 103.7216) (end 134.2898 96.774) (width 1.5) (layer "F.Cu") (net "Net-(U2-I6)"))
 (segment (start 139.9914 85.9416) (end 139.319 86.614) (width 1.5) (layer "F.Cu") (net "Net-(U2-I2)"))
 (segment (start 141.839338 85.9416) (end 139.9914 85.9416) (width 1.5) (layer "F.Cu") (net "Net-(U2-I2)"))
 (segment (start 139.319 86.614) (end 132.842 86.614) (width 1.5) (layer "F.Cu") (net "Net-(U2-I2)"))
 (segment (start 132.842 99.314) (end 133.8326 99.314) (width 1.5) (layer "F.Cu") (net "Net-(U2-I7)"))
 (segment (start 133.8326 99.314) (end 140.7802 106.2616) (width 1.5) (layer "F.Cu") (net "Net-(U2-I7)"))
 (segment (start 140.7802 106.2616) (end 141.839338 106.2616) (width 1.5) (layer "F.Cu") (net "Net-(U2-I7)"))
 (segment (start 139.2054 98.6416) (end 141.839338 98.6416) (width 1.5) (layer "F.Cu") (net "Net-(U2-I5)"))
 (segment (start 132.842 94.234) (end 134.7978 94.234) (width 1.5) (layer "F.Cu") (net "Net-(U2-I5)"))
 (segment (start 134.7978 94.234) (end 139.2054 98.6416) (width 1.5) (layer "F.Cu") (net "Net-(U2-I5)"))
 (segment (start 155.0924 103.808662) (end 165.165338 113.8816) (width 1.5) (layer "F.Cu") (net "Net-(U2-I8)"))
 (segment (start 129.4638 82.3976) (end 130.683 81.1784) (width 1.5) (layer "F.Cu") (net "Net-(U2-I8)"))
 (segment (start 129.4638 100.3758) (end 129.4638 82.3976) (width 1.5) (layer "F.Cu") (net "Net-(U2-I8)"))
 (segment (start 130.942 101.854) (end 129.4638 100.3758) (width 1.5) (layer "F.Cu") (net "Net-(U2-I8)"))
 (segment (start 147.6248 81.1784) (end 155.0924 88.646) (width 1.5) (layer "F.Cu") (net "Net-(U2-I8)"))
 (segment (start 130.683 81.1784) (end 147.6248 81.1784) (width 1.5) (layer "F.Cu") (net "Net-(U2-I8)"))
 (segment (start 155.0924 88.646) (end 155.0924 103.808662) (width 1.5) (layer "F.Cu") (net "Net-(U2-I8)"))
 (segment (start 165.165338 113.8816) (end 167.239338 113.8816) (width 1.5) (layer "F.Cu") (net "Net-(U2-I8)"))
 (segment (start 132.842 101.854) (end 130.942 101.854) (width 1.5) (layer "F.Cu") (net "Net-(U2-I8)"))
 (segment (start 137.4902 84.074) (end 138.2014 83.3628) (width 1.5) (layer "F.Cu") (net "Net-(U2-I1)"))
 (segment (start 138.2402 83.4016) (end 141.839338 83.4016) (width 1.5) (layer "F.Cu") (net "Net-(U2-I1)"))
 (segment (start 132.842 84.074) (end 137.4902 84.074) (width 1.5) (layer "F.Cu") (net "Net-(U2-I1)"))
 (segment (start 138.2014 83.3628) (end 138.2402 83.4016) (width 1.5) (layer "F.Cu") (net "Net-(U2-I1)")))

